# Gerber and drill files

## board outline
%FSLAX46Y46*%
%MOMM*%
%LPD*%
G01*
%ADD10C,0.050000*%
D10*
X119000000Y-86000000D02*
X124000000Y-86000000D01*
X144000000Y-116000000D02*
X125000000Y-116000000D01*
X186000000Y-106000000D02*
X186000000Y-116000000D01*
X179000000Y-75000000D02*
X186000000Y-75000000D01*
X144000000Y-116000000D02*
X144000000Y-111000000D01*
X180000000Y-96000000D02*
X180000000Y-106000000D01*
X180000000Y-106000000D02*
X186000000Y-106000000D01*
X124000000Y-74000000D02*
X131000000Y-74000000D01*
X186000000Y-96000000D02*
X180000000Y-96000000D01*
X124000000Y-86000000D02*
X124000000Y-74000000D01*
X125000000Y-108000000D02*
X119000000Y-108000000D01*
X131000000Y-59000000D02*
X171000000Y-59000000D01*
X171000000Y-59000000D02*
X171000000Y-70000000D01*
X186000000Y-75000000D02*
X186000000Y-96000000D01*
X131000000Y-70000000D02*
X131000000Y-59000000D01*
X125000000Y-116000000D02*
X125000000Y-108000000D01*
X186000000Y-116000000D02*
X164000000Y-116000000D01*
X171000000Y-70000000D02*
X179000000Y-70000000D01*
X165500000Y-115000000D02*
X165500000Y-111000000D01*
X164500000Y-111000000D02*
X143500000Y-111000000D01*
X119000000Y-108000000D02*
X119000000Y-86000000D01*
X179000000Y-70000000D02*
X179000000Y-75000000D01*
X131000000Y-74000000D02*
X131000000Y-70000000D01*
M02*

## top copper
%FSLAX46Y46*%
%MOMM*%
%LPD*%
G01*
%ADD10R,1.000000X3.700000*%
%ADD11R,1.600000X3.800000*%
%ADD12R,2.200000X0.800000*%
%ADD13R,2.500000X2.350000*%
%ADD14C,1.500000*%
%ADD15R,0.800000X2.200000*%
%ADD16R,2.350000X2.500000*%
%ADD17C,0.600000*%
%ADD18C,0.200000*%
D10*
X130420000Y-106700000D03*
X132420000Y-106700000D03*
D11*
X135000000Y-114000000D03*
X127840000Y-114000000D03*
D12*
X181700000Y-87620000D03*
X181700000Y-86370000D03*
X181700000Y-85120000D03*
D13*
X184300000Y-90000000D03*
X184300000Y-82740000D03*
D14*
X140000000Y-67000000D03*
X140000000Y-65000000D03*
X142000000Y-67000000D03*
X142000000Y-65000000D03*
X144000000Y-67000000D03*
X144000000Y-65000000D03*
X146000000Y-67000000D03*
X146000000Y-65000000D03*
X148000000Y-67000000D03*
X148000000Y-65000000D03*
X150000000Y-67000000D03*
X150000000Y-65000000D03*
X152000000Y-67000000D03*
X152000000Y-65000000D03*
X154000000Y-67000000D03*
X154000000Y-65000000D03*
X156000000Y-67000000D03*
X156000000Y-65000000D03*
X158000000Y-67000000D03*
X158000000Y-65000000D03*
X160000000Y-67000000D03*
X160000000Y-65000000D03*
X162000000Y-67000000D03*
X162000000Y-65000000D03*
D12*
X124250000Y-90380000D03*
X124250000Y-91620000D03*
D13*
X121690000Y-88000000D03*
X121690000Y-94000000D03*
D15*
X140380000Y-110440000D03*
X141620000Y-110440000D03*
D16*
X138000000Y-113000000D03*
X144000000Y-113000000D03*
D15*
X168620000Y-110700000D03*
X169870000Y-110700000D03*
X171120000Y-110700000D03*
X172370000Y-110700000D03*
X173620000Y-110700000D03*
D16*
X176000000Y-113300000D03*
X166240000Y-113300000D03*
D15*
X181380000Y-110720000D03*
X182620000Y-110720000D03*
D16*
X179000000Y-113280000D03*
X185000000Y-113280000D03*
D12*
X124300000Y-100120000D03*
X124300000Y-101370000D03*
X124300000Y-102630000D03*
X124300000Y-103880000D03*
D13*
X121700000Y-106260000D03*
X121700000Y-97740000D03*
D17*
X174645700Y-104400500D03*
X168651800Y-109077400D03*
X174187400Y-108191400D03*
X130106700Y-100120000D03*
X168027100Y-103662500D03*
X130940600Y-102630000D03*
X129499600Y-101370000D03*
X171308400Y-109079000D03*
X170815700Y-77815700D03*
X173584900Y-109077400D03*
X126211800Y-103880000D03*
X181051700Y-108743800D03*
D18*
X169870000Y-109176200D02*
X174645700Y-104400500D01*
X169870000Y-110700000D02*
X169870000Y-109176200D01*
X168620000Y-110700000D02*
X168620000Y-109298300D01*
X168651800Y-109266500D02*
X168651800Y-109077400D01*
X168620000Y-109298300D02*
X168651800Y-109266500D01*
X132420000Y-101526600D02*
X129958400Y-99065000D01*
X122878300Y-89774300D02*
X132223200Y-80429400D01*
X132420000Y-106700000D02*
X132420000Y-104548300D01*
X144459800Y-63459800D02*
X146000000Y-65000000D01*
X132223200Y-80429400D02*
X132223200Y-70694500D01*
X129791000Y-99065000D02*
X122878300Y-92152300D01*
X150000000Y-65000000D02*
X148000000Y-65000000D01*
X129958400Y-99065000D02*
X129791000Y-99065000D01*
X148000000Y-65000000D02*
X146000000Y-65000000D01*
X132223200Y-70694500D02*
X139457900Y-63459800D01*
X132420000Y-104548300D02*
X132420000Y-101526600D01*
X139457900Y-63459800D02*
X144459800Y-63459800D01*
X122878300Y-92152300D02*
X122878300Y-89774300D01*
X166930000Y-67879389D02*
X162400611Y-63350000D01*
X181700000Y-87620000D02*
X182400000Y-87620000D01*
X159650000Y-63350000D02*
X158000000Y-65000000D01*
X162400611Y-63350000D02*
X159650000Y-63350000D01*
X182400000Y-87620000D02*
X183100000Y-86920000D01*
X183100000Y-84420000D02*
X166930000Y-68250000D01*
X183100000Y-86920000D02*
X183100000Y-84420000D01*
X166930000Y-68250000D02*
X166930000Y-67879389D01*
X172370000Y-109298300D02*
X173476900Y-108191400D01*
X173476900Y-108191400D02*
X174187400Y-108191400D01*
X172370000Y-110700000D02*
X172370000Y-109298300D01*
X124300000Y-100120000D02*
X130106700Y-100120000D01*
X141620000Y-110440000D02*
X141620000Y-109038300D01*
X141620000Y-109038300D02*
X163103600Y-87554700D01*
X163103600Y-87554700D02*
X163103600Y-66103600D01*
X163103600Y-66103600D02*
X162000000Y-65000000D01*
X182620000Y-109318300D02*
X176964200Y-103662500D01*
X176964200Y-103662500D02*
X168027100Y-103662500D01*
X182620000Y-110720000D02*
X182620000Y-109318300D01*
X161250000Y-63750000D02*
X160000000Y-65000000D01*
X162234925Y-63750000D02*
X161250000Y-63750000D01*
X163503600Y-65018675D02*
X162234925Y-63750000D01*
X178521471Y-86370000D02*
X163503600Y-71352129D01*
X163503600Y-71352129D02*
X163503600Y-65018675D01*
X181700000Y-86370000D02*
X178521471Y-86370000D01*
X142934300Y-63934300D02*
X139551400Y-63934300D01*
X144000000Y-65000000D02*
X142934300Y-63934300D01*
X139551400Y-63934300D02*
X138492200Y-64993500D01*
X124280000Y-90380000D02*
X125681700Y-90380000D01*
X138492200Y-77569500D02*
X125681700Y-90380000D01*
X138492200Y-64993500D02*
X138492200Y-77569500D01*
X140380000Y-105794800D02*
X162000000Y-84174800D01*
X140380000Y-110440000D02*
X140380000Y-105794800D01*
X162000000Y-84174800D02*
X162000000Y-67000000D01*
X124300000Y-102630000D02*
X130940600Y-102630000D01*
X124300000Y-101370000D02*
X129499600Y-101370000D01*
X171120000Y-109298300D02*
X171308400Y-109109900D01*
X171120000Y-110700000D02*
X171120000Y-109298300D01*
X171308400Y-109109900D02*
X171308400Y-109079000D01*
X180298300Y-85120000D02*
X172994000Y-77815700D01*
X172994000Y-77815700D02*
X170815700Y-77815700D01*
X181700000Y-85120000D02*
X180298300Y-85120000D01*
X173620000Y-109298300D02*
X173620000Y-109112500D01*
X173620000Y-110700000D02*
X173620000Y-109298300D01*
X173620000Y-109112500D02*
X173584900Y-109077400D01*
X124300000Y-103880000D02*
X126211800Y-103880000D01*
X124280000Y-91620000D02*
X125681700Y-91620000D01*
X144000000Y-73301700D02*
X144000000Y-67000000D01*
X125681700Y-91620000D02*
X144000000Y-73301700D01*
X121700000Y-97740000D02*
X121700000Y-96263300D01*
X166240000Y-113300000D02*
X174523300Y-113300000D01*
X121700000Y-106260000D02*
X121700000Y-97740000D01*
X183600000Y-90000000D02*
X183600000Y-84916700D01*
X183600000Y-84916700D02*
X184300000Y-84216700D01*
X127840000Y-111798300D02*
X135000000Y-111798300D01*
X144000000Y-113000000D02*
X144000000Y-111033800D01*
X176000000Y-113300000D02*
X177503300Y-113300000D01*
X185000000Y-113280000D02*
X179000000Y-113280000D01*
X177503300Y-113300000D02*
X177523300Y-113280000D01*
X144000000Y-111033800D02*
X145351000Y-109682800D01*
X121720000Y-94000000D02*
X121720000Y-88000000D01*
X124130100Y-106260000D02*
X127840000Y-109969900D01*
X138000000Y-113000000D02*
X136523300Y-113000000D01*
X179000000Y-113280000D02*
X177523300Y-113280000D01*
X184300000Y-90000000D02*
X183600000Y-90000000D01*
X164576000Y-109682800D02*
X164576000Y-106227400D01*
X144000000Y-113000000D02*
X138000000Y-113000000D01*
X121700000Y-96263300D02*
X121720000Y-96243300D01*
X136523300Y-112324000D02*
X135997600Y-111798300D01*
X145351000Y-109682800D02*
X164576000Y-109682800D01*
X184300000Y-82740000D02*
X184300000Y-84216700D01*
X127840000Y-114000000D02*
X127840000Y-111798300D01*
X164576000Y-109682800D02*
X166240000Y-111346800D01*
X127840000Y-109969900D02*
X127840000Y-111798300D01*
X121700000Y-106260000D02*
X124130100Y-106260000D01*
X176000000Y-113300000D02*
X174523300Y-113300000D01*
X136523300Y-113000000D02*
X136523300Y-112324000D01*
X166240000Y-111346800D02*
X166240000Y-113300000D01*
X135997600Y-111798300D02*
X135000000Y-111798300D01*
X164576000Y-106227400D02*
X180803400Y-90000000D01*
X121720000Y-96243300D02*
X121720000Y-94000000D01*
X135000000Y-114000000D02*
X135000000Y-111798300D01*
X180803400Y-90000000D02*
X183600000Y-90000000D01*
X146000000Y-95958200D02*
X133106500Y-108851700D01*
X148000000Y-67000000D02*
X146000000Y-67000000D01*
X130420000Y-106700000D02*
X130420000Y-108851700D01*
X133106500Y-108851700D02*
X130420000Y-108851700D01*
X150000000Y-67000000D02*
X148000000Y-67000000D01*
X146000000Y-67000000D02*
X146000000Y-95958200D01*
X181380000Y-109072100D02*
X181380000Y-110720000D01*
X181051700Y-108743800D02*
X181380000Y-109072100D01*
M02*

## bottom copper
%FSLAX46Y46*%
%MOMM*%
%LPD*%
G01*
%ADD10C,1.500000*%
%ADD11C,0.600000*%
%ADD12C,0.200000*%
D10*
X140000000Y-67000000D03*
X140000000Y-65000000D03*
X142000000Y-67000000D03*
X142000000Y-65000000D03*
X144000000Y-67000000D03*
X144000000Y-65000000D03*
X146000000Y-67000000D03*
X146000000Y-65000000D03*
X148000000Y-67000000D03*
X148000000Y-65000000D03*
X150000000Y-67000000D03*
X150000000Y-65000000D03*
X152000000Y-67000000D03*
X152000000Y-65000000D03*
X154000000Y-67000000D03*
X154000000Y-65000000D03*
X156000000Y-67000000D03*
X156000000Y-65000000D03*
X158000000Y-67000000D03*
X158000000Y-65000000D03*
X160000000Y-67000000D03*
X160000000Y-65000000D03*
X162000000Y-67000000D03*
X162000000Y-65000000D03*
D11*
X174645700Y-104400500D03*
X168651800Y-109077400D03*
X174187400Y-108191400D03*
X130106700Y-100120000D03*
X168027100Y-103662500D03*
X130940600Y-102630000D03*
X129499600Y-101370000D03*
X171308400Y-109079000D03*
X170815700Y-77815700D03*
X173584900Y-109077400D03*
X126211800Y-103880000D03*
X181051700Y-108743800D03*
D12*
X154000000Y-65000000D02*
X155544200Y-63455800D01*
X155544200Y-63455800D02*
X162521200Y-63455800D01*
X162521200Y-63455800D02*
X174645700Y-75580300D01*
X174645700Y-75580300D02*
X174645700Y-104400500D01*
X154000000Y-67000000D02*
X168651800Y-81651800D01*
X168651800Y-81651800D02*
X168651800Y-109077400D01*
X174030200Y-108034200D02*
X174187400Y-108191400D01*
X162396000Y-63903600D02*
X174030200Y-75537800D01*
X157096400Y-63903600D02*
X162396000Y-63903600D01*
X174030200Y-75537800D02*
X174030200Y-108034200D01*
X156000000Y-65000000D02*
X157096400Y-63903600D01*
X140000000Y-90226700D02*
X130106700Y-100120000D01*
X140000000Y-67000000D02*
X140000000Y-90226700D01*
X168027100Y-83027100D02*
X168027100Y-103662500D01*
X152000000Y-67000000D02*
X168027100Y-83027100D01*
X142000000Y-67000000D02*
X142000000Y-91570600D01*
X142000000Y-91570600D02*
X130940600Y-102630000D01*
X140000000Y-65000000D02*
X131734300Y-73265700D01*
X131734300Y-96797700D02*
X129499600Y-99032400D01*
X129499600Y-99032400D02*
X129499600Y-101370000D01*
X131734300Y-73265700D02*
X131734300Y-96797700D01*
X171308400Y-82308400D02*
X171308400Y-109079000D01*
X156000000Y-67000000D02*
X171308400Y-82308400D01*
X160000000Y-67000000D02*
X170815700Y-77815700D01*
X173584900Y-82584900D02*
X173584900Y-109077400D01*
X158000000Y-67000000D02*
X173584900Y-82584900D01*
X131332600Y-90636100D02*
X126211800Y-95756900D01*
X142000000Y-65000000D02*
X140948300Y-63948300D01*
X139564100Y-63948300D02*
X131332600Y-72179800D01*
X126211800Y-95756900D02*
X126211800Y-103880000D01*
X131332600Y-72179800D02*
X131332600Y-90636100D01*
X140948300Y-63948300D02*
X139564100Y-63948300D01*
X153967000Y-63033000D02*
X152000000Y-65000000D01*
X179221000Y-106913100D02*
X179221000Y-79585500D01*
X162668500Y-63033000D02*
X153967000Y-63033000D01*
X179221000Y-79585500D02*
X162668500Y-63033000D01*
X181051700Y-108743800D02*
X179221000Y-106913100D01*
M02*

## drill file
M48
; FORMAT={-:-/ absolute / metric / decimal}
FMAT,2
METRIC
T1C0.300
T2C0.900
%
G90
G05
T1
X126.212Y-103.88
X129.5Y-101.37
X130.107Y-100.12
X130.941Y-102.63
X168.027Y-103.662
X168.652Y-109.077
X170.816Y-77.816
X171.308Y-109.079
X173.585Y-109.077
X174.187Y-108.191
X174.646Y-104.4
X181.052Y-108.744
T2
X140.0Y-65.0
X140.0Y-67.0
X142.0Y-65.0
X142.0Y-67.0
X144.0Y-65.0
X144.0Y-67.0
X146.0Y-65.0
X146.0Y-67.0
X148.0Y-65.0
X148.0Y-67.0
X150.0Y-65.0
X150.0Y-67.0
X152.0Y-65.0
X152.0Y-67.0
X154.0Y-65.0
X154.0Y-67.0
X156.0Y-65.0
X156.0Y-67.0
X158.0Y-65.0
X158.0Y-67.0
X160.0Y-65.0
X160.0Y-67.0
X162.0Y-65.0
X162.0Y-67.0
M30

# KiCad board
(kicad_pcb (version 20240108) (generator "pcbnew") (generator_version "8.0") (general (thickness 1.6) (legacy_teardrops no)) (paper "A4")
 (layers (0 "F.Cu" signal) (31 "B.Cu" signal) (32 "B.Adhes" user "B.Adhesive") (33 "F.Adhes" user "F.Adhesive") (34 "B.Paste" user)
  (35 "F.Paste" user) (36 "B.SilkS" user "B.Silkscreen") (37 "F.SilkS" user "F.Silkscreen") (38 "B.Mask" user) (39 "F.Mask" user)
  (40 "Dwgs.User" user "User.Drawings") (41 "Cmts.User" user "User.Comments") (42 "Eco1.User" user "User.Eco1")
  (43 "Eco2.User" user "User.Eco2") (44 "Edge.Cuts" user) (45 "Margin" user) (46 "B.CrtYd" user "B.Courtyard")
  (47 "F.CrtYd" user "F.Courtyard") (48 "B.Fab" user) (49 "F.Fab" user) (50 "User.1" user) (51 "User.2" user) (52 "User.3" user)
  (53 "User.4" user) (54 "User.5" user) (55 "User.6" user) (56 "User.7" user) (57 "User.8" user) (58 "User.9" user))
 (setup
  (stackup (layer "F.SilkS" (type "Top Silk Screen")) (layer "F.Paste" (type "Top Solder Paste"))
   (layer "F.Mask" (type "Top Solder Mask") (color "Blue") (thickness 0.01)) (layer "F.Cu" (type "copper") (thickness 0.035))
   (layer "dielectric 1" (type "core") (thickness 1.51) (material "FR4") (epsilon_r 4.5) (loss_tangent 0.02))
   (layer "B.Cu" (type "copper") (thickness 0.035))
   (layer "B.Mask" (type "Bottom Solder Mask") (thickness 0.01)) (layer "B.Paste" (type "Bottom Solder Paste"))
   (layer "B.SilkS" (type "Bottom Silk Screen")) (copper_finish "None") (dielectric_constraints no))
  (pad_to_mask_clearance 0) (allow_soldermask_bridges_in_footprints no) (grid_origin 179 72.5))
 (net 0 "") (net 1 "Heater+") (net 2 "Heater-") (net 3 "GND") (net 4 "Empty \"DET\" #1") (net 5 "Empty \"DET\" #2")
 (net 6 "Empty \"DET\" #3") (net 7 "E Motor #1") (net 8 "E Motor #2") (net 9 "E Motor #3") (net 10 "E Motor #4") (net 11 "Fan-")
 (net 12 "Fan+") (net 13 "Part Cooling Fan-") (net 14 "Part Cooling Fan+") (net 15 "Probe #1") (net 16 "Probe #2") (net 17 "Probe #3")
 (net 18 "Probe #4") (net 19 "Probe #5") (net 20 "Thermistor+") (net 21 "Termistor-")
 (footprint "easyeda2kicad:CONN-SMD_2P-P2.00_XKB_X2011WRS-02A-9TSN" (layer "F.Cu") (at 131.42 110.35)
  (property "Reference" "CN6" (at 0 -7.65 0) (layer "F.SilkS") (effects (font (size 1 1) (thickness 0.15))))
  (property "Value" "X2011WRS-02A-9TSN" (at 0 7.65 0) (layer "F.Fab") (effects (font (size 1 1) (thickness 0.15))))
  (pad "1" smd rect (at -1 -3.65) (size 1 3.7) (layers "F.Cu" "F.Paste" "F.Mask") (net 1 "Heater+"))
  (pad "2" smd rect (at 1 -3.65) (size 1 3.7) (layers "F.Cu" "F.Paste" "F.Mask") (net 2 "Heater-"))
  (pad "3" smd rect (at 3.58 3.65) (size 1.6 3.8) (layers "F.Cu" "F.Paste" "F.Mask") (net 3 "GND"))
  (pad "4" smd rect (at -3.58 3.65) (size 1.6 3.8) (layers "F.Cu" "F.Paste" "F.Mask") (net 3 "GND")))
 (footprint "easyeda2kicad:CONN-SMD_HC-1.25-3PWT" (layer "F.Cu") (at 183 86.37 90)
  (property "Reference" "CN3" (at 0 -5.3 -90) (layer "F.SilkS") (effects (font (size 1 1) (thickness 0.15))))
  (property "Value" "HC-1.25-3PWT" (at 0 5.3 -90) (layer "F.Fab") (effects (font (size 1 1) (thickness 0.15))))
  (pad "1" smd rect (at -1.25 -1.3 90) (size 0.8 2.2) (layers "F.Cu" "F.Paste" "F.Mask") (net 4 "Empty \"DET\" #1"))
  (pad "2" smd rect (at 0 -1.3 90) (size 0.8 2.2) (layers "F.Cu" "F.Paste" "F.Mask") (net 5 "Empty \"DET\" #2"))
  (pad "3" smd rect (at 1.25 -1.3 90) (size 0.8 2.2) (layers "F.Cu" "F.Paste" "F.Mask") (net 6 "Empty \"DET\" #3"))
  (pad "4" smd rect (at -3.63 1.3 90) (size 2.35 2.5) (layers "F.Cu" "F.Paste" "F.Mask") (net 3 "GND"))
  (pad "5" smd rect (at 3.63 1.3 90) (size 2.35 2.5) (layers "F.Cu" "F.Paste" "F.Mask") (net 3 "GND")))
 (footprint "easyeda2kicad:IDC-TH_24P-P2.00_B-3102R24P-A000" (layer "F.Cu") (at 151 66 180)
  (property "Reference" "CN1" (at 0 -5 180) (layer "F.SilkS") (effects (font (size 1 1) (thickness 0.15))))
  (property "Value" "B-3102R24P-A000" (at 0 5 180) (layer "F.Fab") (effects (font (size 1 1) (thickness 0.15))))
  (pad "1" thru_hole circle (at 11 -1 90) (size 1.5 1.5) (drill 0.900024) (layers "*.Cu" "*.Mask") (remove_unused_layers no)
   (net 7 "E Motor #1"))
  (pad "2" thru_hole circle (at 11 1 90) (size 1.5 1.5) (drill 0.900024) (layers "*.Cu" "*.Mask") (remove_unused_layers no)
   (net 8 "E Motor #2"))
  (pad "3" thru_hole circle (at 9 -1 90) (size 1.5 1.5) (drill 0.900024) (layers "*.Cu" "*.Mask") (remove_unused_layers no)
   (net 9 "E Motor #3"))
  (pad "4" thru_hole circle (at 9 1 90) (size 1.5 1.5) (drill 0.900024) (layers "*.Cu" "*.Mask") (remove_unused_layers no)
   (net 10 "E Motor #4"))
  (pad "5" thru_hole circle (at 7 -1 90) (size 1.5 1.5) (drill 0.900024) (layers "*.Cu" "*.Mask") (remove_unused_layers no) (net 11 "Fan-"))
  (pad "6" thru_hole circle (at 7 1 90) (size 1.5 1.5) (drill 0.900024) (layers "*.Cu" "*.Mask") (remove_unused_layers no) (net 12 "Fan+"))
  (pad "7" thru_hole circle (at 5 -1 90) (size 1.5 1.5) (drill 0.900024) (layers "*.Cu" "*.Mask") (remove_unused_layers no)
   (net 1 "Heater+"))
  (pad "8" thru_hole circle (at 5 1 90) (size 1.5 1.5) (drill 0.900024) (layers "*.Cu" "*.Mask") (remove_unused_layers no) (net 2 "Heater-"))
  (pad "9" thru_hole circle (at 3 -1 90) (size 1.5 1.5) (drill 0.900024) (layers "*.Cu" "*.Mask") (remove_unused_layers no)
   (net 1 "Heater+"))
  (pad "10" thru_hole circle (at 3 1 90) (size 1.5 1.5) (drill 0.900024) (layers "*.Cu" "*.Mask") (remove_unused_layers no)
   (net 2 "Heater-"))
  (pad "11" thru_hole circle (at 1 -1 90) (size 1.5 1.5) (drill 0.900024) (layers "*.Cu" "*.Mask") (remove_unused_layers no)
   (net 1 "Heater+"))
  (pad "12" thru_hole circle (at 1 1 90) (size 1.5 1.5) (drill 0.900024) (layers "*.Cu" "*.Mask") (remove_unused_layers no)
   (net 2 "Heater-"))
  (pad "13" thru_hole circle (at -1 -1 90) (size 1.5 1.5) (drill 0.900024) (layers "*.Cu" "*.Mask") (remove_unused_layers no)
   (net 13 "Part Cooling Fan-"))
  (pad "14" thru_hole circle (at -1 1 90) (size 1.5 1.5) (drill 0.900024) (layers "*.Cu" "*.Mask") (remove_unused_layers no)
   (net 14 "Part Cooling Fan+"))
  (pad "15" thru_hole circle (at -3 -1 90) (size 1.5 1.5) (drill 0.900024) (layers "*.Cu" "*.Mask") (remove_unused_layers no)
   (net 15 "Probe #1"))
  (pad "16" thru_hole circle (at -3 1 90) (size 1.5 1.5) (drill 0.900024) (layers "*.Cu" "*.Mask") (remove_unused_layers no)
   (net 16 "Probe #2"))
  (pad "17" thru_hole circle (at -5 -1 90) (size 1.5 1.5) (drill 0.900024) (layers "*.Cu" "*.Mask") (remove_unused_layers no)
   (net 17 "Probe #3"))
  (pad "18" thru_hole circle (at -5 1 90) (size 1.5 1.5) (drill 0.900024) (layers "*.Cu" "*.Mask") (remove_unused_layers no)
   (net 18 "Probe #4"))
  (pad "19" thru_hole circle (at -7 -1 90) (size 1.5 1.5) (drill 0.900024) (layers "*.Cu" "*.Mask") (remove_unused_layers no)
   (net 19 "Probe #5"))
  (pad "20" thru_hole circle (at -7 1 90) (size 1.5 1.5) (drill 0.900024) (layers "*.Cu" "*.Mask") (remove_unused_layers no)
   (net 4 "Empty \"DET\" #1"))
  (pad "21" thru_hole circle (at -9 -1 90) (size 1.5 1.5) (drill 0.900024) (layers "*.Cu" "*.Mask") (remove_unused_layers no)
   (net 6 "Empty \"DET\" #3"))
  (pad "22" thru_hole circle (at -9 1 90) (size 1.5 1.5) (drill 0.900024) (layers "*.Cu" "*.Mask") (remove_unused_layers no)
   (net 5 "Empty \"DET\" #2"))
  (pad "23" thru_hole circle (at -11 -1 90) (size 1.5 1.5) (drill 0.900024) (layers "*.Cu" "*.Mask") (remove_unused_layers no)
   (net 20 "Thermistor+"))
  (pad "24" thru_hole circle (at -11 1 90) (size 1.5 1.5) (drill 0.900024) (layers "*.Cu" "*.Mask") (remove_unused_layers no)
   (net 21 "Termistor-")))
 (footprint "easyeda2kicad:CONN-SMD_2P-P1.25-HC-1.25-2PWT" (layer "F.Cu") (at 122.97 91 -90)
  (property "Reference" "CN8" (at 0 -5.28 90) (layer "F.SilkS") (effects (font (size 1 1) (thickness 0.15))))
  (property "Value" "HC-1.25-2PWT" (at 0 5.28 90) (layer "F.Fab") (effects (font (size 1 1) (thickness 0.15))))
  (pad "1" smd rect (at -0.62 -1.28 270) (size 0.8 2.2) (layers "F.Cu" "F.Paste" "F.Mask") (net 12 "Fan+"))
  (pad "2" smd rect (at 0.62 -1.28 270) (size 0.8 2.2) (layers "F.Cu" "F.Paste" "F.Mask") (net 11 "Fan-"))
  (pad "3" smd rect (at -3 1.28 180) (size 2.5 2.35) (layers "F.Cu" "F.Paste" "F.Mask") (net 3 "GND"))
  (pad "4" smd rect (at 3 1.28) (size 2.5 2.35) (layers "F.Cu" "F.Paste" "F.Mask") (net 3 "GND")))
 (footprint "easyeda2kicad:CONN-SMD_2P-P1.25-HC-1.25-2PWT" (layer "F.Cu") (at 141 111.72)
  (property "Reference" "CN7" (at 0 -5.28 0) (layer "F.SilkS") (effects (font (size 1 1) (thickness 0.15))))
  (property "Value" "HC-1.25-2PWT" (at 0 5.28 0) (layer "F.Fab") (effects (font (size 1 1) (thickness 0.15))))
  (pad "1" smd rect (at -0.62 -1.28) (size 0.8 2.2) (layers "F.Cu" "F.Paste" "F.Mask") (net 20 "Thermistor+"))
  (pad "2" smd rect (at 0.62 -1.28) (size 0.8 2.2) (layers "F.Cu" "F.Paste" "F.Mask") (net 21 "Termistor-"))
  (pad "3" smd rect (at -3 1.28 270) (size 2.5 2.35) (layers "F.Cu" "F.Paste" "F.Mask") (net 3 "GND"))
  (pad "4" smd rect (at 3 1.28 90) (size 2.5 2.35) (layers "F.Cu" "F.Paste" "F.Mask") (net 3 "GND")))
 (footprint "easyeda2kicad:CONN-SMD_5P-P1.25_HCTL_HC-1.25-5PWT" (layer "F.Cu") (at 171.12 112)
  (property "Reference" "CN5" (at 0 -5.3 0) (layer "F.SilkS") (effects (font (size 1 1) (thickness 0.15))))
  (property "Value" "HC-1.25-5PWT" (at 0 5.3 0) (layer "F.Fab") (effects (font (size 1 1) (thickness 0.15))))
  (pad "1" smd rect (at -2.5 -1.3) (size 0.8 2.2) (layers "F.Cu" "F.Paste" "F.Mask") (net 15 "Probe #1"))
  (pad "2" smd rect (at -1.25 -1.3) (size 0.8 2.2) (layers "F.Cu" "F.Paste" "F.Mask") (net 16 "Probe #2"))
  (pad "3" smd rect (at 0 -1.3) (size 0.8 2.2) (layers "F.Cu" "F.Paste" "F.Mask") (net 17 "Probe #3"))
  (pad "4" smd rect (at 1.25 -1.3) (size 0.8 2.2) (layers "F.Cu" "F.Paste" "F.Mask") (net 18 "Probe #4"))
  (pad "5" smd rect (at 2.5 -1.3) (size 0.8 2.2) (layers "F.Cu" "F.Paste" "F.Mask") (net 19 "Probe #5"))
  (pad "6" smd rect (at 4.88 1.3) (size 2.35 2.5) (layers "F.Cu" "F.Paste" "F.Mask") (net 3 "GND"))
  (pad "7" smd rect (at -4.88 1.3) (size 2.35 2.5) (layers "F.Cu" "F.Paste" "F.Mask") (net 3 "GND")))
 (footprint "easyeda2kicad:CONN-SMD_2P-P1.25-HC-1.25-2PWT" (layer "F.Cu") (at 182 112)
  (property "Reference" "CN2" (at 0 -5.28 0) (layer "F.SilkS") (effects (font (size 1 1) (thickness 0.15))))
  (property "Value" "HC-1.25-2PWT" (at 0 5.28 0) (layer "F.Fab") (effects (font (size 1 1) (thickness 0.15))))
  (pad "1" smd rect (at -0.62 -1.28) (size 0.8 2.2) (layers "F.Cu" "F.Paste" "F.Mask") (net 14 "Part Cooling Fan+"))
  (pad "2" smd rect (at 0.62 -1.28) (size 0.8 2.2) (layers "F.Cu" "F.Paste" "F.Mask") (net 13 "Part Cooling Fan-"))
  (pad "3" smd rect (at -3 1.28 270) (size 2.5 2.35) (layers "F.Cu" "F.Paste" "F.Mask") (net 3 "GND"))
  (pad "4" smd rect (at 3 1.28 90) (size 2.5 2.35) (layers "F.Cu" "F.Paste" "F.Mask") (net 3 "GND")))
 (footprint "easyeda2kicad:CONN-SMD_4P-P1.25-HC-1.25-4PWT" (layer "F.Cu") (at 123 102 -90)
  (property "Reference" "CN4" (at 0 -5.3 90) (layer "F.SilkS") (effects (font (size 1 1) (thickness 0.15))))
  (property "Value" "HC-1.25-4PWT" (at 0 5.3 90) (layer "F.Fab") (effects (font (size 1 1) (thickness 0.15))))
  (pad "1" smd rect (at -1.88 -1.3) (size 2.2 0.8) (layers "F.Cu" "F.Paste" "F.Mask") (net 7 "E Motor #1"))
  (pad "2" smd rect (at -0.63 -1.3) (size 2.2 0.8) (layers "F.Cu" "F.Paste" "F.Mask") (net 8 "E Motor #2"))
  (pad "3" smd rect (at 0.63 -1.3) (size 2.2 0.8) (layers "F.Cu" "F.Paste" "F.Mask") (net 9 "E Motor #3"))
  (pad "4" smd rect (at 1.88 -1.3) (size 2.2 0.8) (layers "F.Cu" "F.Paste" "F.Mask") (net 10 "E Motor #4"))
  (pad "5" smd rect (at 4.26 1.3 90) (size 2.35 2.5) (layers "F.Cu" "F.Paste" "F.Mask") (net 3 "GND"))
  (pad "6" smd rect (at -4.26 1.3 90) (size 2.35 2.5) (layers "F.Cu" "F.Paste" "F.Mask") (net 3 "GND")))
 (gr_line (start 119 86) (end 124 86) (stroke (width 0.05) (type default)) (layer "Edge.Cuts"))
 (gr_line (start 144 116) (end 125 116) (stroke (width 0.05) (type default)) (layer "Edge.Cuts"))
 (gr_line (start 186 106) (end 186 116) (stroke (width 0.05) (type default)) (layer "Edge.Cuts"))
 (gr_line (start 179 75) (end 186 75) (stroke (width 0.05) (type default)) (layer "Edge.Cuts"))
 (gr_line (start 144 116) (end 144 111) (stroke (width 0.05) (type default)) (layer "Edge.Cuts"))
 (gr_line (start 180 96) (end 180 106) (stroke (width 0.05) (type default)) (layer "Edge.Cuts"))
 (gr_line (start 180 106) (end 186 106) (stroke (width 0.05) (type default)) (layer "Edge.Cuts"))
 (gr_line (start 124 74) (end 131 74) (stroke (width 0.05) (type default)) (layer "Edge.Cuts"))
 (gr_line (start 186 96) (end 180 96) (stroke (width 0.05) (type default)) (layer "Edge.Cuts"))
 (gr_line (start 124 86) (end 124 74) (stroke (width 0.05) (type default)) (layer "Edge.Cuts"))
 (gr_line (start 125 108) (end 119 108) (stroke (width 0.05) (type default)) (layer "Edge.Cuts"))
 (gr_line (start 131 59) (end 171 59) (stroke (width 0.05) (type default)) (layer "Edge.Cuts"))
 (gr_line (start 171 59) (end 171 70) (stroke (width 0.05) (type default)) (layer "Edge.Cuts"))
 (gr_line (start 186 75) (end 186 96) (stroke (width 0.05) (type default)) (layer "Edge.Cuts"))
 (gr_line (start 131 70) (end 131 59) (stroke (width 0.05) (type default)) (layer "Edge.Cuts"))
 (gr_line (start 125 116) (end 125 108) (stroke (width 0.05) (type default)) (layer "Edge.Cuts"))
 (gr_line (start 186 116) (end 164 116) (stroke (width 0.05) (type default)) (layer "Edge.Cuts"))
 (gr_line (start 171 70) (end 179 70) (stroke (width 0.05) (type default)) (layer "Edge.Cuts"))
 (gr_line (start 165.5 115) (end 165.5 111) (stroke (width 0.05) (type default)) (layer "Edge.Cuts"))
 (gr_line (start 164.5 111) (end 143.5 111) (stroke (width 0.05) (type default)) (layer "Edge.Cuts"))
 (gr_line (start 119 108) (end 119 86) (stroke (width 0.05) (type default)) (layer "Edge.Cuts"))
 (gr_line (start 179 70) (end 179 75) (stroke (width 0.05) (type default)) (layer "Edge.Cuts"))
 (gr_line (start 131 74) (end 131 70) (stroke (width 0.05) (type default)) (layer "Edge.Cuts"))
 (segment (start 169.87 109.1762) (end 174.6457 104.4005) (width 0.2) (layer "F.Cu") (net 16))
 (segment (start 169.87 110.7) (end 169.87 109.1762) (width 0.2) (layer "F.Cu") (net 16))
 (via (at 174.6457 104.4005) (size 0.6) (drill 0.3) (layers "F.Cu" "B.Cu") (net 16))
 (segment (start 154 65) (end 155.5442 63.4558) (width 0.2) (layer "B.Cu") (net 16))
 (segment (start 155.5442 63.4558) (end 162.5212 63.4558) (width 0.2) (layer "B.Cu") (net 16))
 (segment (start 162.5212 63.4558) (end 174.6457 75.5803) (width 0.2) (layer "B.Cu") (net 16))
 (segment (start 174.6457 75.5803) (end 174.6457 104.4005) (width 0.2) (layer "B.Cu") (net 16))
 (segment (start 168.62 110.7) (end 168.62 109.2983) (width 0.2) (layer "F.Cu") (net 15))
 (segment (start 168.6518 109.2665) (end 168.6518 109.0774) (width 0.2) (layer "F.Cu") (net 15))
 (segment (start 168.62 109.2983) (end 168.6518 109.2665) (width 0.2) (layer "F.Cu") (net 15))
 (via (at 168.6518 109.0774) (size 0.6) (drill 0.3) (layers "F.Cu" "B.Cu") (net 15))
 (segment (start 154 67) (end 168.6518 81.6518) (width 0.2) (layer "B.Cu") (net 15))
 (segment (start 168.6518 81.6518) (end 168.6518 109.0774) (width 0.2) (layer "B.Cu") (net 15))
 (segment (start 132.42 101.5266) (end 129.9584 99.065) (width 0.2) (layer "F.Cu") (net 2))
 (segment (start 122.8783 89.7743) (end 132.2232 80.4294) (width 0.2) (layer "F.Cu") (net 2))
 (segment (start 132.42 106.7) (end 132.42 104.5483) (width 0.2) (layer "F.Cu") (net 2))
 (segment (start 144.4598 63.4598) (end 146 65) (width 0.2) (layer "F.Cu") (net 2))
 (segment (start 132.2232 80.4294) (end 132.2232 70.6945) (width 0.2) (layer "F.Cu") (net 2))
 (segment (start 129.791 99.065) (end 122.8783 92.1523) (width 0.2) (layer "F.Cu") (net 2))
 (segment (start 150 65) (end 148 65) (width 0.2) (layer "F.Cu") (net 2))
 (segment (start 129.9584 99.065) (end 129.791 99.065) (width 0.2) (layer "F.Cu") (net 2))
 (segment (start 148 65) (end 146 65) (width 0.2) (layer "F.Cu") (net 2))
 (segment (start 132.2232 70.6945) (end 139.4579 63.4598) (width 0.2) (layer "F.Cu") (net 2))
 (segment (start 132.42 104.5483) (end 132.42 101.5266) (width 0.2) (layer "F.Cu") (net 2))
 (segment (start 139.4579 63.4598) (end 144.4598 63.4598) (width 0.2) (layer "F.Cu") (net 2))
 (segment (start 122.8783 92.1523) (end 122.8783 89.7743) (width 0.2) (layer "F.Cu") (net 2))
 (segment (start 166.93 67.879389) (end 162.400611 63.35) (width 0.2) (layer "F.Cu") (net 4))
 (segment (start 181.7 87.62) (end 182.4 87.62) (width 0.2) (layer "F.Cu") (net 4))
 (segment (start 159.65 63.35) (end 158 65) (width 0.2) (layer "F.Cu") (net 4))
 (segment (start 162.400611 63.35) (end 159.65 63.35) (width 0.2) (layer "F.Cu") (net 4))
 (segment (start 182.4 87.62) (end 183.1 86.92) (width 0.2) (layer "F.Cu") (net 4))
 (segment (start 183.1 84.42) (end 166.93 68.25) (width 0.2) (layer "F.Cu") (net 4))
 (segment (start 183.1 86.92) (end 183.1 84.42) (width 0.2) (layer "F.Cu") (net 4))
 (segment (start 166.93 68.25) (end 166.93 67.879389) (width 0.2) (layer "F.Cu") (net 4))
 (segment (start 172.37 109.2983) (end 173.4769 108.1914) (width 0.2) (layer "F.Cu") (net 18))
 (segment (start 173.4769 108.1914) (end 174.1874 108.1914) (width 0.2) (layer "F.Cu") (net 18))
 (segment (start 172.37 110.7) (end 172.37 109.2983) (width 0.2) (layer "F.Cu") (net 18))
 (via (at 174.1874 108.1914) (size 0.6) (drill 0.3) (layers "F.Cu" "B.Cu") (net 18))
 (segment (start 174.0302 108.0342) (end 174.1874 108.1914) (width 0.2) (layer "B.Cu") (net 18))
 (segment (start 162.396 63.9036) (end 174.0302 75.5378) (width 0.2) (layer "B.Cu") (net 18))
 (segment (start 157.0964 63.9036) (end 162.396 63.9036) (width 0.2) (layer "B.Cu") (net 18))
 (segment (start 174.0302 75.5378) (end 174.0302 108.0342) (width 0.2) (layer "B.Cu") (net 18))
 (segment (start 156 65) (end 157.0964 63.9036) (width 0.2) (layer "B.Cu") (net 18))
 (segment (start 124.3 100.12) (end 130.1067 100.12) (width 0.2) (layer "F.Cu") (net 7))
 (via (at 130.1067 100.12) (size 0.6) (drill 0.3) (layers "F.Cu" "B.Cu") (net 7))
 (segment (start 140 90.2267) (end 130.1067 100.12) (width 0.2) (layer "B.Cu") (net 7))
 (segment (start 140 67) (end 140 90.2267) (width 0.2) (layer "B.Cu") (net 7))
 (segment (start 141.62 110.44) (end 141.62 109.0383) (width 0.2) (layer "F.Cu") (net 21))
 (segment (start 141.62 109.0383) (end 163.1036 87.5547) (width 0.2) (layer "F.Cu") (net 21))
 (segment (start 163.1036 87.5547) (end 163.1036 66.1036) (width 0.2) (layer "F.Cu") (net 21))
 (segment (start 163.1036 66.1036) (end 162 65) (width 0.2) (layer "F.Cu") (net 21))
 (segment (start 182.62 109.3183) (end 176.9642 103.6625) (width 0.2) (layer "F.Cu") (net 13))
 (segment (start 176.9642 103.6625) (end 168.0271 103.6625) (width 0.2) (layer "F.Cu") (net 13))
 (segment (start 182.62 110.72) (end 182.62 109.3183) (width 0.2) (layer "F.Cu") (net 13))
 (via (at 168.0271 103.6625) (size 0.6) (drill 0.3) (layers "F.Cu" "B.Cu") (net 13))
 (segment (start 168.0271 83.0271) (end 168.0271 103.6625) (width 0.2) (layer "B.Cu") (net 13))
 (segment (start 152 67) (end 168.0271 83.0271) (width 0.2) (layer "B.Cu") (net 13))
 (segment (start 161.25 63.75) (end 160 65) (width 0.2) (layer "F.Cu") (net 5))
 (segment (start 162.234925 63.75) (end 161.25 63.75) (width 0.2) (layer "F.Cu") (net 5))
 (segment (start 163.5036 65.018675) (end 162.234925 63.75) (width 0.2) (layer "F.Cu") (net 5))
 (segment (start 178.521471 86.37) (end 163.5036 71.352129) (width 0.2) (layer "F.Cu") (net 5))
 (segment (start 163.5036 71.352129) (end 163.5036 65.018675) (width 0.2) (layer "F.Cu") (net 5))
 (segment (start 181.7 86.37) (end 178.521471 86.37) (width 0.2) (layer "F.Cu") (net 5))
 (segment (start 142.9343 63.9343) (end 139.5514 63.9343) (width 0.2) (layer "F.Cu") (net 12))
 (segment (start 144 65) (end 142.9343 63.9343) (width 0.2) (layer "F.Cu") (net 12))
 (segment (start 139.5514 63.9343) (end 138.4922 64.9935) (width 0.2) (layer "F.Cu") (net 12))
 (segment (start 124.28 90.38) (end 125.6817 90.38) (width 0.2) (layer "F.Cu") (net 12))
 (segment (start 138.4922 77.5695) (end 125.6817 90.38) (width 0.2) (layer "F.Cu") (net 12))
 (segment (start 138.4922 64.9935) (end 138.4922 77.5695) (width 0.2) (layer "F.Cu") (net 12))
 (segment (start 140.38 105.7948) (end 162 84.1748) (width 0.2) (layer "F.Cu") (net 20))
 (segment (start 140.38 110.44) (end 140.38 105.7948) (width 0.2) (layer "F.Cu") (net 20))
 (segment (start 162 84.1748) (end 162 67) (width 0.2) (layer "F.Cu") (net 20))
 (segment (start 124.3 102.63) (end 130.9406 102.63) (width 0.2) (layer "F.Cu") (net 9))
 (via (at 130.9406 102.63) (size 0.6) (drill 0.3) (layers "F.Cu" "B.Cu") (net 9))
 (segment (start 142 67) (end 142 91.5706) (width 0.2) (layer "B.Cu") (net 9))
 (segment (start 142 91.5706) (end 130.9406 102.63) (width 0.2) (layer "B.Cu") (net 9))
 (segment (start 124.3 101.37) (end 129.4996 101.37) (width 0.2) (layer "F.Cu") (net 8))
 (via (at 129.4996 101.37) (size 0.6) (drill 0.3) (layers "F.Cu" "B.Cu") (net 8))
 (segment (start 140 65) (end 131.7343 73.2657) (width 0.2) (layer "B.Cu") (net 8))
 (segment (start 131.7343 96.7977) (end 129.4996 99.0324) (width 0.2) (layer "B.Cu") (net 8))
 (segment (start 129.4996 99.0324) (end 129.4996 101.37) (width 0.2) (layer "B.Cu") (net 8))
 (segment (start 131.7343 73.2657) (end 131.7343 96.7977) (width 0.2) (layer "B.Cu") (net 8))
 (segment (start 171.12 109.2983) (end 171.3084 109.1099) (width 0.2) (layer "F.Cu") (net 17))
 (segment (start 171.12 110.7) (end 171.12 109.2983) (width 0.2) (layer "F.Cu") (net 17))
 (segment (start 171.3084 109.1099) (end 171.3084 109.079) (width 0.2) (layer "F.Cu") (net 17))
 (via (at 171.3084 109.079) (size 0.6) (drill 0.3) (layers "F.Cu" "B.Cu") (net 17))
 (segment (start 171.3084 82.3084) (end 171.3084 109.079) (width 0.2) (layer "B.Cu") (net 17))
 (segment (start 156 67) (end 171.3084 82.3084) (width 0.2) (layer "B.Cu") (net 17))
 (segment (start 180.2983 85.12) (end 172.994 77.8157) (width 0.2) (layer "F.Cu") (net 6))
 (segment (start 172.994 77.8157) (end 170.8157 77.8157) (width 0.2) (layer "F.Cu") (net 6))
 (segment (start 181.7 85.12) (end 180.2983 85.12) (width 0.2) (layer "F.Cu") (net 6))
 (via (at 170.8157 77.8157) (size 0.6) (drill 0.3) (layers "F.Cu" "B.Cu") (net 6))
 (segment (start 160 67) (end 170.8157 77.8157) (width 0.2) (layer "B.Cu") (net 6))
 (segment (start 173.62 109.2983) (end 173.62 109.1125) (width 0.2) (layer "F.Cu") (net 19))
 (segment (start 173.62 110.7) (end 173.62 109.2983) (width 0.2) (layer "F.Cu") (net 19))
 (segment (start 173.62 109.1125) (end 173.5849 109.0774) (width 0.2) (layer "F.Cu") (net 19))
 (via (at 173.5849 109.0774) (size 0.6) (drill 0.3) (layers "F.Cu" "B.Cu") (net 19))
 (segment (start 173.5849 82.5849) (end 173.5849 109.0774) (width 0.2) (layer "B.Cu") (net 19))
 (segment (start 158 67) (end 173.5849 82.5849) (width 0.2) (layer "B.Cu") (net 19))
 (segment (start 124.3 103.88) (end 126.2118 103.88) (width 0.2) (layer "F.Cu") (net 10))
 (via (at 126.2118 103.88) (size 0.6) (drill 0.3) (layers "F.Cu" "B.Cu") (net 10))
 (segment (start 131.3326 90.6361) (end 126.2118 95.7569) (width 0.2) (layer "B.Cu") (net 10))
 (segment (start 142 65) (end 140.9483 63.9483) (width 0.2) (layer "B.Cu") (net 10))
 (segment (start 139.5641 63.9483) (end 131.3326 72.1798) (width 0.2) (layer "B.Cu") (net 10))
 (segment (start 126.2118 95.7569) (end 126.2118 103.88) (width 0.2) (layer "B.Cu") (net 10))
 (segment (start 131.3326 72.1798) (end 131.3326 90.6361) (width 0.2) (layer "B.Cu") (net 10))
 (segment (start 140.9483 63.9483) (end 139.5641 63.9483) (width 0.2) (layer "B.Cu") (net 10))
 (segment (start 124.28 91.62) (end 125.6817 91.62) (width 0.2) (layer "F.Cu") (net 11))
 (segment (start 144 73.3017) (end 144 67) (width 0.2) (layer "F.Cu") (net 11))
 (segment (start 125.6817 91.62) (end 144 73.3017) (width 0.2) (layer "F.Cu") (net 11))
 (segment (start 121.7 97.74) (end 121.7 96.2633) (width 0.2) (layer "F.Cu") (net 3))
 (segment (start 166.24 113.3) (end 174.5233 113.3) (width 0.2) (layer "F.Cu") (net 3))
 (segment (start 121.7 106.26) (end 121.7 97.74) (width 0.2) (layer "F.Cu") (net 3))
 (segment (start 183.6 90) (end 183.6 84.9167) (width 0.2) (layer "F.Cu") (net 3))
 (segment (start 183.6 84.9167) (end 184.3 84.2167) (width 0.2) (layer "F.Cu") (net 3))
 (segment (start 127.84 111.7983) (end 135 111.7983) (width 0.2) (layer "F.Cu") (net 3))
 (segment (start 144 113) (end 144 111.0338) (width 0.2) (layer "F.Cu") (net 3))
 (segment (start 176 113.3) (end 177.5033 113.3) (width 0.2) (layer "F.Cu") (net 3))
 (segment (start 185 113.28) (end 179 113.28) (width 0.2) (layer "F.Cu") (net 3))
 (segment (start 177.5033 113.3) (end 177.5233 113.28) (width 0.2) (layer "F.Cu") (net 3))
 (segment (start 144 111.0338) (end 145.351 109.6828) (width 0.2) (layer "F.Cu") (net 3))
 (segment (start 121.72 94) (end 121.72 88) (width 0.2) (layer "F.Cu") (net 3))
 (segment (start 124.1301 106.26) (end 127.84 109.9699) (width 0.2) (layer "F.Cu") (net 3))
 (segment (start 138 113) (end 136.5233 113) (width 0.2) (layer "F.Cu") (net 3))
 (segment (start 179 113.28) (end 177.5233 113.28) (width 0.2) (layer "F.Cu") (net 3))
 (segment (start 184.3 90) (end 183.6 90) (width 0.2) (layer "F.Cu") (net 3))
 (segment (start 164.576 109.6828) (end 164.576 106.2274) (width 0.2) (layer "F.Cu") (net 3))
 (segment (start 144 113) (end 138 113) (width 0.2) (layer "F.Cu") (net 3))
 (segment (start 121.7 96.2633) (end 121.72 96.2433) (width 0.2) (layer "F.Cu") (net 3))
 (segment (start 136.5233 112.324) (end 135.9976 111.7983) (width 0.2) (layer "F.Cu") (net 3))
 (segment (start 145.351 109.6828) (end 164.576 109.6828) (width 0.2) (layer "F.Cu") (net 3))
 (segment (start 184.3 82.74) (end 184.3 84.2167) (width 0.2) (layer "F.Cu") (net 3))
 (segment (start 127.84 114) (end 127.84 111.7983) (width 0.2) (layer "F.Cu") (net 3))
 (segment (start 164.576 109.6828) (end 166.24 111.3468) (width 0.2) (layer "F.Cu") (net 3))
 (segment (start 127.84 109.9699) (end 127.84 111.7983) (width 0.2) (layer "F.Cu") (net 3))
 (segment (start 121.7 106.26) (end 124.1301 106.26) (width 0.2) (layer "F.Cu") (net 3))
 (segment (start 176 113.3) (end 174.5233 113.3) (width 0.2) (layer "F.Cu") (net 3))
 (segment (start 136.5233 113) (end 136.5233 112.324) (width 0.2) (layer "F.Cu") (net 3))
 (segment (start 166.24 111.3468) (end 166.24 113.3) (width 0.2) (layer "F.Cu") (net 3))
 (segment (start 135.9976 111.7983) (end 135 111.7983) (width 0.2) (layer "F.Cu") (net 3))
 (segment (start 164.576 106.2274) (end 180.8034 90) (width 0.2) (layer "F.Cu") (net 3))
 (segment (start 121.72 96.2433) (end 121.72 94) (width 0.2) (layer "F.Cu") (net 3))
 (segment (start 135 114) (end 135 111.7983) (width 0.2) (layer "F.Cu") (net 3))
 (segment (start 180.8034 90) (end 183.6 90) (width 0.2) (layer "F.Cu") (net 3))
 (segment (start 146 95.9582) (end 133.1065 108.8517) (width 0.2) (layer "F.Cu") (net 1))
 (segment (start 148 67) (end 146 67) (width 0.2) (layer "F.Cu") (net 1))
 (segment (start 130.42 106.7) (end 130.42 108.8517) (width 0.2) (layer "F.Cu") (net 1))
 (segment (start 133.1065 108.8517) (end 130.42 108.8517) (width 0.2) (layer "F.Cu") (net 1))
 (segment (start 150 67) (end 148 67) (width 0.2) (layer "F.Cu") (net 1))
 (segment (start 146 67) (end 146 95.9582) (width 0.2) (layer "F.Cu") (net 1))
 (segment (start 181.38 109.0721) (end 181.38 110.72) (width 0.2) (layer "F.Cu") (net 14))
 (segment (start 181.0517 108.7438) (end 181.38 109.0721) (width 0.2) (layer "F.Cu") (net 14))
 (via (at 181.0517 108.7438) (size 0.6) (drill 0.3) (layers "F.Cu" "B.Cu") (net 14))
 (segment (start 153.967 63.033) (end 152 65) (width 0.2) (layer "B.Cu") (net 14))
 (segment (start 179.221 106.9131) (end 179.221 79.5855) (width 0.2) (layer "B.Cu") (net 14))
 (segment (start 162.6685 63.033) (end 153.967 63.033) (width 0.2) (layer "B.Cu") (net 14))
 (segment (start 179.221 79.5855) (end 162.6685 63.033) (width 0.2) (layer "B.Cu") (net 14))
 (segment (start 181.0517 108.7438) (end 179.221 106.9131) (width 0.2) (layer "B.Cu") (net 14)))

